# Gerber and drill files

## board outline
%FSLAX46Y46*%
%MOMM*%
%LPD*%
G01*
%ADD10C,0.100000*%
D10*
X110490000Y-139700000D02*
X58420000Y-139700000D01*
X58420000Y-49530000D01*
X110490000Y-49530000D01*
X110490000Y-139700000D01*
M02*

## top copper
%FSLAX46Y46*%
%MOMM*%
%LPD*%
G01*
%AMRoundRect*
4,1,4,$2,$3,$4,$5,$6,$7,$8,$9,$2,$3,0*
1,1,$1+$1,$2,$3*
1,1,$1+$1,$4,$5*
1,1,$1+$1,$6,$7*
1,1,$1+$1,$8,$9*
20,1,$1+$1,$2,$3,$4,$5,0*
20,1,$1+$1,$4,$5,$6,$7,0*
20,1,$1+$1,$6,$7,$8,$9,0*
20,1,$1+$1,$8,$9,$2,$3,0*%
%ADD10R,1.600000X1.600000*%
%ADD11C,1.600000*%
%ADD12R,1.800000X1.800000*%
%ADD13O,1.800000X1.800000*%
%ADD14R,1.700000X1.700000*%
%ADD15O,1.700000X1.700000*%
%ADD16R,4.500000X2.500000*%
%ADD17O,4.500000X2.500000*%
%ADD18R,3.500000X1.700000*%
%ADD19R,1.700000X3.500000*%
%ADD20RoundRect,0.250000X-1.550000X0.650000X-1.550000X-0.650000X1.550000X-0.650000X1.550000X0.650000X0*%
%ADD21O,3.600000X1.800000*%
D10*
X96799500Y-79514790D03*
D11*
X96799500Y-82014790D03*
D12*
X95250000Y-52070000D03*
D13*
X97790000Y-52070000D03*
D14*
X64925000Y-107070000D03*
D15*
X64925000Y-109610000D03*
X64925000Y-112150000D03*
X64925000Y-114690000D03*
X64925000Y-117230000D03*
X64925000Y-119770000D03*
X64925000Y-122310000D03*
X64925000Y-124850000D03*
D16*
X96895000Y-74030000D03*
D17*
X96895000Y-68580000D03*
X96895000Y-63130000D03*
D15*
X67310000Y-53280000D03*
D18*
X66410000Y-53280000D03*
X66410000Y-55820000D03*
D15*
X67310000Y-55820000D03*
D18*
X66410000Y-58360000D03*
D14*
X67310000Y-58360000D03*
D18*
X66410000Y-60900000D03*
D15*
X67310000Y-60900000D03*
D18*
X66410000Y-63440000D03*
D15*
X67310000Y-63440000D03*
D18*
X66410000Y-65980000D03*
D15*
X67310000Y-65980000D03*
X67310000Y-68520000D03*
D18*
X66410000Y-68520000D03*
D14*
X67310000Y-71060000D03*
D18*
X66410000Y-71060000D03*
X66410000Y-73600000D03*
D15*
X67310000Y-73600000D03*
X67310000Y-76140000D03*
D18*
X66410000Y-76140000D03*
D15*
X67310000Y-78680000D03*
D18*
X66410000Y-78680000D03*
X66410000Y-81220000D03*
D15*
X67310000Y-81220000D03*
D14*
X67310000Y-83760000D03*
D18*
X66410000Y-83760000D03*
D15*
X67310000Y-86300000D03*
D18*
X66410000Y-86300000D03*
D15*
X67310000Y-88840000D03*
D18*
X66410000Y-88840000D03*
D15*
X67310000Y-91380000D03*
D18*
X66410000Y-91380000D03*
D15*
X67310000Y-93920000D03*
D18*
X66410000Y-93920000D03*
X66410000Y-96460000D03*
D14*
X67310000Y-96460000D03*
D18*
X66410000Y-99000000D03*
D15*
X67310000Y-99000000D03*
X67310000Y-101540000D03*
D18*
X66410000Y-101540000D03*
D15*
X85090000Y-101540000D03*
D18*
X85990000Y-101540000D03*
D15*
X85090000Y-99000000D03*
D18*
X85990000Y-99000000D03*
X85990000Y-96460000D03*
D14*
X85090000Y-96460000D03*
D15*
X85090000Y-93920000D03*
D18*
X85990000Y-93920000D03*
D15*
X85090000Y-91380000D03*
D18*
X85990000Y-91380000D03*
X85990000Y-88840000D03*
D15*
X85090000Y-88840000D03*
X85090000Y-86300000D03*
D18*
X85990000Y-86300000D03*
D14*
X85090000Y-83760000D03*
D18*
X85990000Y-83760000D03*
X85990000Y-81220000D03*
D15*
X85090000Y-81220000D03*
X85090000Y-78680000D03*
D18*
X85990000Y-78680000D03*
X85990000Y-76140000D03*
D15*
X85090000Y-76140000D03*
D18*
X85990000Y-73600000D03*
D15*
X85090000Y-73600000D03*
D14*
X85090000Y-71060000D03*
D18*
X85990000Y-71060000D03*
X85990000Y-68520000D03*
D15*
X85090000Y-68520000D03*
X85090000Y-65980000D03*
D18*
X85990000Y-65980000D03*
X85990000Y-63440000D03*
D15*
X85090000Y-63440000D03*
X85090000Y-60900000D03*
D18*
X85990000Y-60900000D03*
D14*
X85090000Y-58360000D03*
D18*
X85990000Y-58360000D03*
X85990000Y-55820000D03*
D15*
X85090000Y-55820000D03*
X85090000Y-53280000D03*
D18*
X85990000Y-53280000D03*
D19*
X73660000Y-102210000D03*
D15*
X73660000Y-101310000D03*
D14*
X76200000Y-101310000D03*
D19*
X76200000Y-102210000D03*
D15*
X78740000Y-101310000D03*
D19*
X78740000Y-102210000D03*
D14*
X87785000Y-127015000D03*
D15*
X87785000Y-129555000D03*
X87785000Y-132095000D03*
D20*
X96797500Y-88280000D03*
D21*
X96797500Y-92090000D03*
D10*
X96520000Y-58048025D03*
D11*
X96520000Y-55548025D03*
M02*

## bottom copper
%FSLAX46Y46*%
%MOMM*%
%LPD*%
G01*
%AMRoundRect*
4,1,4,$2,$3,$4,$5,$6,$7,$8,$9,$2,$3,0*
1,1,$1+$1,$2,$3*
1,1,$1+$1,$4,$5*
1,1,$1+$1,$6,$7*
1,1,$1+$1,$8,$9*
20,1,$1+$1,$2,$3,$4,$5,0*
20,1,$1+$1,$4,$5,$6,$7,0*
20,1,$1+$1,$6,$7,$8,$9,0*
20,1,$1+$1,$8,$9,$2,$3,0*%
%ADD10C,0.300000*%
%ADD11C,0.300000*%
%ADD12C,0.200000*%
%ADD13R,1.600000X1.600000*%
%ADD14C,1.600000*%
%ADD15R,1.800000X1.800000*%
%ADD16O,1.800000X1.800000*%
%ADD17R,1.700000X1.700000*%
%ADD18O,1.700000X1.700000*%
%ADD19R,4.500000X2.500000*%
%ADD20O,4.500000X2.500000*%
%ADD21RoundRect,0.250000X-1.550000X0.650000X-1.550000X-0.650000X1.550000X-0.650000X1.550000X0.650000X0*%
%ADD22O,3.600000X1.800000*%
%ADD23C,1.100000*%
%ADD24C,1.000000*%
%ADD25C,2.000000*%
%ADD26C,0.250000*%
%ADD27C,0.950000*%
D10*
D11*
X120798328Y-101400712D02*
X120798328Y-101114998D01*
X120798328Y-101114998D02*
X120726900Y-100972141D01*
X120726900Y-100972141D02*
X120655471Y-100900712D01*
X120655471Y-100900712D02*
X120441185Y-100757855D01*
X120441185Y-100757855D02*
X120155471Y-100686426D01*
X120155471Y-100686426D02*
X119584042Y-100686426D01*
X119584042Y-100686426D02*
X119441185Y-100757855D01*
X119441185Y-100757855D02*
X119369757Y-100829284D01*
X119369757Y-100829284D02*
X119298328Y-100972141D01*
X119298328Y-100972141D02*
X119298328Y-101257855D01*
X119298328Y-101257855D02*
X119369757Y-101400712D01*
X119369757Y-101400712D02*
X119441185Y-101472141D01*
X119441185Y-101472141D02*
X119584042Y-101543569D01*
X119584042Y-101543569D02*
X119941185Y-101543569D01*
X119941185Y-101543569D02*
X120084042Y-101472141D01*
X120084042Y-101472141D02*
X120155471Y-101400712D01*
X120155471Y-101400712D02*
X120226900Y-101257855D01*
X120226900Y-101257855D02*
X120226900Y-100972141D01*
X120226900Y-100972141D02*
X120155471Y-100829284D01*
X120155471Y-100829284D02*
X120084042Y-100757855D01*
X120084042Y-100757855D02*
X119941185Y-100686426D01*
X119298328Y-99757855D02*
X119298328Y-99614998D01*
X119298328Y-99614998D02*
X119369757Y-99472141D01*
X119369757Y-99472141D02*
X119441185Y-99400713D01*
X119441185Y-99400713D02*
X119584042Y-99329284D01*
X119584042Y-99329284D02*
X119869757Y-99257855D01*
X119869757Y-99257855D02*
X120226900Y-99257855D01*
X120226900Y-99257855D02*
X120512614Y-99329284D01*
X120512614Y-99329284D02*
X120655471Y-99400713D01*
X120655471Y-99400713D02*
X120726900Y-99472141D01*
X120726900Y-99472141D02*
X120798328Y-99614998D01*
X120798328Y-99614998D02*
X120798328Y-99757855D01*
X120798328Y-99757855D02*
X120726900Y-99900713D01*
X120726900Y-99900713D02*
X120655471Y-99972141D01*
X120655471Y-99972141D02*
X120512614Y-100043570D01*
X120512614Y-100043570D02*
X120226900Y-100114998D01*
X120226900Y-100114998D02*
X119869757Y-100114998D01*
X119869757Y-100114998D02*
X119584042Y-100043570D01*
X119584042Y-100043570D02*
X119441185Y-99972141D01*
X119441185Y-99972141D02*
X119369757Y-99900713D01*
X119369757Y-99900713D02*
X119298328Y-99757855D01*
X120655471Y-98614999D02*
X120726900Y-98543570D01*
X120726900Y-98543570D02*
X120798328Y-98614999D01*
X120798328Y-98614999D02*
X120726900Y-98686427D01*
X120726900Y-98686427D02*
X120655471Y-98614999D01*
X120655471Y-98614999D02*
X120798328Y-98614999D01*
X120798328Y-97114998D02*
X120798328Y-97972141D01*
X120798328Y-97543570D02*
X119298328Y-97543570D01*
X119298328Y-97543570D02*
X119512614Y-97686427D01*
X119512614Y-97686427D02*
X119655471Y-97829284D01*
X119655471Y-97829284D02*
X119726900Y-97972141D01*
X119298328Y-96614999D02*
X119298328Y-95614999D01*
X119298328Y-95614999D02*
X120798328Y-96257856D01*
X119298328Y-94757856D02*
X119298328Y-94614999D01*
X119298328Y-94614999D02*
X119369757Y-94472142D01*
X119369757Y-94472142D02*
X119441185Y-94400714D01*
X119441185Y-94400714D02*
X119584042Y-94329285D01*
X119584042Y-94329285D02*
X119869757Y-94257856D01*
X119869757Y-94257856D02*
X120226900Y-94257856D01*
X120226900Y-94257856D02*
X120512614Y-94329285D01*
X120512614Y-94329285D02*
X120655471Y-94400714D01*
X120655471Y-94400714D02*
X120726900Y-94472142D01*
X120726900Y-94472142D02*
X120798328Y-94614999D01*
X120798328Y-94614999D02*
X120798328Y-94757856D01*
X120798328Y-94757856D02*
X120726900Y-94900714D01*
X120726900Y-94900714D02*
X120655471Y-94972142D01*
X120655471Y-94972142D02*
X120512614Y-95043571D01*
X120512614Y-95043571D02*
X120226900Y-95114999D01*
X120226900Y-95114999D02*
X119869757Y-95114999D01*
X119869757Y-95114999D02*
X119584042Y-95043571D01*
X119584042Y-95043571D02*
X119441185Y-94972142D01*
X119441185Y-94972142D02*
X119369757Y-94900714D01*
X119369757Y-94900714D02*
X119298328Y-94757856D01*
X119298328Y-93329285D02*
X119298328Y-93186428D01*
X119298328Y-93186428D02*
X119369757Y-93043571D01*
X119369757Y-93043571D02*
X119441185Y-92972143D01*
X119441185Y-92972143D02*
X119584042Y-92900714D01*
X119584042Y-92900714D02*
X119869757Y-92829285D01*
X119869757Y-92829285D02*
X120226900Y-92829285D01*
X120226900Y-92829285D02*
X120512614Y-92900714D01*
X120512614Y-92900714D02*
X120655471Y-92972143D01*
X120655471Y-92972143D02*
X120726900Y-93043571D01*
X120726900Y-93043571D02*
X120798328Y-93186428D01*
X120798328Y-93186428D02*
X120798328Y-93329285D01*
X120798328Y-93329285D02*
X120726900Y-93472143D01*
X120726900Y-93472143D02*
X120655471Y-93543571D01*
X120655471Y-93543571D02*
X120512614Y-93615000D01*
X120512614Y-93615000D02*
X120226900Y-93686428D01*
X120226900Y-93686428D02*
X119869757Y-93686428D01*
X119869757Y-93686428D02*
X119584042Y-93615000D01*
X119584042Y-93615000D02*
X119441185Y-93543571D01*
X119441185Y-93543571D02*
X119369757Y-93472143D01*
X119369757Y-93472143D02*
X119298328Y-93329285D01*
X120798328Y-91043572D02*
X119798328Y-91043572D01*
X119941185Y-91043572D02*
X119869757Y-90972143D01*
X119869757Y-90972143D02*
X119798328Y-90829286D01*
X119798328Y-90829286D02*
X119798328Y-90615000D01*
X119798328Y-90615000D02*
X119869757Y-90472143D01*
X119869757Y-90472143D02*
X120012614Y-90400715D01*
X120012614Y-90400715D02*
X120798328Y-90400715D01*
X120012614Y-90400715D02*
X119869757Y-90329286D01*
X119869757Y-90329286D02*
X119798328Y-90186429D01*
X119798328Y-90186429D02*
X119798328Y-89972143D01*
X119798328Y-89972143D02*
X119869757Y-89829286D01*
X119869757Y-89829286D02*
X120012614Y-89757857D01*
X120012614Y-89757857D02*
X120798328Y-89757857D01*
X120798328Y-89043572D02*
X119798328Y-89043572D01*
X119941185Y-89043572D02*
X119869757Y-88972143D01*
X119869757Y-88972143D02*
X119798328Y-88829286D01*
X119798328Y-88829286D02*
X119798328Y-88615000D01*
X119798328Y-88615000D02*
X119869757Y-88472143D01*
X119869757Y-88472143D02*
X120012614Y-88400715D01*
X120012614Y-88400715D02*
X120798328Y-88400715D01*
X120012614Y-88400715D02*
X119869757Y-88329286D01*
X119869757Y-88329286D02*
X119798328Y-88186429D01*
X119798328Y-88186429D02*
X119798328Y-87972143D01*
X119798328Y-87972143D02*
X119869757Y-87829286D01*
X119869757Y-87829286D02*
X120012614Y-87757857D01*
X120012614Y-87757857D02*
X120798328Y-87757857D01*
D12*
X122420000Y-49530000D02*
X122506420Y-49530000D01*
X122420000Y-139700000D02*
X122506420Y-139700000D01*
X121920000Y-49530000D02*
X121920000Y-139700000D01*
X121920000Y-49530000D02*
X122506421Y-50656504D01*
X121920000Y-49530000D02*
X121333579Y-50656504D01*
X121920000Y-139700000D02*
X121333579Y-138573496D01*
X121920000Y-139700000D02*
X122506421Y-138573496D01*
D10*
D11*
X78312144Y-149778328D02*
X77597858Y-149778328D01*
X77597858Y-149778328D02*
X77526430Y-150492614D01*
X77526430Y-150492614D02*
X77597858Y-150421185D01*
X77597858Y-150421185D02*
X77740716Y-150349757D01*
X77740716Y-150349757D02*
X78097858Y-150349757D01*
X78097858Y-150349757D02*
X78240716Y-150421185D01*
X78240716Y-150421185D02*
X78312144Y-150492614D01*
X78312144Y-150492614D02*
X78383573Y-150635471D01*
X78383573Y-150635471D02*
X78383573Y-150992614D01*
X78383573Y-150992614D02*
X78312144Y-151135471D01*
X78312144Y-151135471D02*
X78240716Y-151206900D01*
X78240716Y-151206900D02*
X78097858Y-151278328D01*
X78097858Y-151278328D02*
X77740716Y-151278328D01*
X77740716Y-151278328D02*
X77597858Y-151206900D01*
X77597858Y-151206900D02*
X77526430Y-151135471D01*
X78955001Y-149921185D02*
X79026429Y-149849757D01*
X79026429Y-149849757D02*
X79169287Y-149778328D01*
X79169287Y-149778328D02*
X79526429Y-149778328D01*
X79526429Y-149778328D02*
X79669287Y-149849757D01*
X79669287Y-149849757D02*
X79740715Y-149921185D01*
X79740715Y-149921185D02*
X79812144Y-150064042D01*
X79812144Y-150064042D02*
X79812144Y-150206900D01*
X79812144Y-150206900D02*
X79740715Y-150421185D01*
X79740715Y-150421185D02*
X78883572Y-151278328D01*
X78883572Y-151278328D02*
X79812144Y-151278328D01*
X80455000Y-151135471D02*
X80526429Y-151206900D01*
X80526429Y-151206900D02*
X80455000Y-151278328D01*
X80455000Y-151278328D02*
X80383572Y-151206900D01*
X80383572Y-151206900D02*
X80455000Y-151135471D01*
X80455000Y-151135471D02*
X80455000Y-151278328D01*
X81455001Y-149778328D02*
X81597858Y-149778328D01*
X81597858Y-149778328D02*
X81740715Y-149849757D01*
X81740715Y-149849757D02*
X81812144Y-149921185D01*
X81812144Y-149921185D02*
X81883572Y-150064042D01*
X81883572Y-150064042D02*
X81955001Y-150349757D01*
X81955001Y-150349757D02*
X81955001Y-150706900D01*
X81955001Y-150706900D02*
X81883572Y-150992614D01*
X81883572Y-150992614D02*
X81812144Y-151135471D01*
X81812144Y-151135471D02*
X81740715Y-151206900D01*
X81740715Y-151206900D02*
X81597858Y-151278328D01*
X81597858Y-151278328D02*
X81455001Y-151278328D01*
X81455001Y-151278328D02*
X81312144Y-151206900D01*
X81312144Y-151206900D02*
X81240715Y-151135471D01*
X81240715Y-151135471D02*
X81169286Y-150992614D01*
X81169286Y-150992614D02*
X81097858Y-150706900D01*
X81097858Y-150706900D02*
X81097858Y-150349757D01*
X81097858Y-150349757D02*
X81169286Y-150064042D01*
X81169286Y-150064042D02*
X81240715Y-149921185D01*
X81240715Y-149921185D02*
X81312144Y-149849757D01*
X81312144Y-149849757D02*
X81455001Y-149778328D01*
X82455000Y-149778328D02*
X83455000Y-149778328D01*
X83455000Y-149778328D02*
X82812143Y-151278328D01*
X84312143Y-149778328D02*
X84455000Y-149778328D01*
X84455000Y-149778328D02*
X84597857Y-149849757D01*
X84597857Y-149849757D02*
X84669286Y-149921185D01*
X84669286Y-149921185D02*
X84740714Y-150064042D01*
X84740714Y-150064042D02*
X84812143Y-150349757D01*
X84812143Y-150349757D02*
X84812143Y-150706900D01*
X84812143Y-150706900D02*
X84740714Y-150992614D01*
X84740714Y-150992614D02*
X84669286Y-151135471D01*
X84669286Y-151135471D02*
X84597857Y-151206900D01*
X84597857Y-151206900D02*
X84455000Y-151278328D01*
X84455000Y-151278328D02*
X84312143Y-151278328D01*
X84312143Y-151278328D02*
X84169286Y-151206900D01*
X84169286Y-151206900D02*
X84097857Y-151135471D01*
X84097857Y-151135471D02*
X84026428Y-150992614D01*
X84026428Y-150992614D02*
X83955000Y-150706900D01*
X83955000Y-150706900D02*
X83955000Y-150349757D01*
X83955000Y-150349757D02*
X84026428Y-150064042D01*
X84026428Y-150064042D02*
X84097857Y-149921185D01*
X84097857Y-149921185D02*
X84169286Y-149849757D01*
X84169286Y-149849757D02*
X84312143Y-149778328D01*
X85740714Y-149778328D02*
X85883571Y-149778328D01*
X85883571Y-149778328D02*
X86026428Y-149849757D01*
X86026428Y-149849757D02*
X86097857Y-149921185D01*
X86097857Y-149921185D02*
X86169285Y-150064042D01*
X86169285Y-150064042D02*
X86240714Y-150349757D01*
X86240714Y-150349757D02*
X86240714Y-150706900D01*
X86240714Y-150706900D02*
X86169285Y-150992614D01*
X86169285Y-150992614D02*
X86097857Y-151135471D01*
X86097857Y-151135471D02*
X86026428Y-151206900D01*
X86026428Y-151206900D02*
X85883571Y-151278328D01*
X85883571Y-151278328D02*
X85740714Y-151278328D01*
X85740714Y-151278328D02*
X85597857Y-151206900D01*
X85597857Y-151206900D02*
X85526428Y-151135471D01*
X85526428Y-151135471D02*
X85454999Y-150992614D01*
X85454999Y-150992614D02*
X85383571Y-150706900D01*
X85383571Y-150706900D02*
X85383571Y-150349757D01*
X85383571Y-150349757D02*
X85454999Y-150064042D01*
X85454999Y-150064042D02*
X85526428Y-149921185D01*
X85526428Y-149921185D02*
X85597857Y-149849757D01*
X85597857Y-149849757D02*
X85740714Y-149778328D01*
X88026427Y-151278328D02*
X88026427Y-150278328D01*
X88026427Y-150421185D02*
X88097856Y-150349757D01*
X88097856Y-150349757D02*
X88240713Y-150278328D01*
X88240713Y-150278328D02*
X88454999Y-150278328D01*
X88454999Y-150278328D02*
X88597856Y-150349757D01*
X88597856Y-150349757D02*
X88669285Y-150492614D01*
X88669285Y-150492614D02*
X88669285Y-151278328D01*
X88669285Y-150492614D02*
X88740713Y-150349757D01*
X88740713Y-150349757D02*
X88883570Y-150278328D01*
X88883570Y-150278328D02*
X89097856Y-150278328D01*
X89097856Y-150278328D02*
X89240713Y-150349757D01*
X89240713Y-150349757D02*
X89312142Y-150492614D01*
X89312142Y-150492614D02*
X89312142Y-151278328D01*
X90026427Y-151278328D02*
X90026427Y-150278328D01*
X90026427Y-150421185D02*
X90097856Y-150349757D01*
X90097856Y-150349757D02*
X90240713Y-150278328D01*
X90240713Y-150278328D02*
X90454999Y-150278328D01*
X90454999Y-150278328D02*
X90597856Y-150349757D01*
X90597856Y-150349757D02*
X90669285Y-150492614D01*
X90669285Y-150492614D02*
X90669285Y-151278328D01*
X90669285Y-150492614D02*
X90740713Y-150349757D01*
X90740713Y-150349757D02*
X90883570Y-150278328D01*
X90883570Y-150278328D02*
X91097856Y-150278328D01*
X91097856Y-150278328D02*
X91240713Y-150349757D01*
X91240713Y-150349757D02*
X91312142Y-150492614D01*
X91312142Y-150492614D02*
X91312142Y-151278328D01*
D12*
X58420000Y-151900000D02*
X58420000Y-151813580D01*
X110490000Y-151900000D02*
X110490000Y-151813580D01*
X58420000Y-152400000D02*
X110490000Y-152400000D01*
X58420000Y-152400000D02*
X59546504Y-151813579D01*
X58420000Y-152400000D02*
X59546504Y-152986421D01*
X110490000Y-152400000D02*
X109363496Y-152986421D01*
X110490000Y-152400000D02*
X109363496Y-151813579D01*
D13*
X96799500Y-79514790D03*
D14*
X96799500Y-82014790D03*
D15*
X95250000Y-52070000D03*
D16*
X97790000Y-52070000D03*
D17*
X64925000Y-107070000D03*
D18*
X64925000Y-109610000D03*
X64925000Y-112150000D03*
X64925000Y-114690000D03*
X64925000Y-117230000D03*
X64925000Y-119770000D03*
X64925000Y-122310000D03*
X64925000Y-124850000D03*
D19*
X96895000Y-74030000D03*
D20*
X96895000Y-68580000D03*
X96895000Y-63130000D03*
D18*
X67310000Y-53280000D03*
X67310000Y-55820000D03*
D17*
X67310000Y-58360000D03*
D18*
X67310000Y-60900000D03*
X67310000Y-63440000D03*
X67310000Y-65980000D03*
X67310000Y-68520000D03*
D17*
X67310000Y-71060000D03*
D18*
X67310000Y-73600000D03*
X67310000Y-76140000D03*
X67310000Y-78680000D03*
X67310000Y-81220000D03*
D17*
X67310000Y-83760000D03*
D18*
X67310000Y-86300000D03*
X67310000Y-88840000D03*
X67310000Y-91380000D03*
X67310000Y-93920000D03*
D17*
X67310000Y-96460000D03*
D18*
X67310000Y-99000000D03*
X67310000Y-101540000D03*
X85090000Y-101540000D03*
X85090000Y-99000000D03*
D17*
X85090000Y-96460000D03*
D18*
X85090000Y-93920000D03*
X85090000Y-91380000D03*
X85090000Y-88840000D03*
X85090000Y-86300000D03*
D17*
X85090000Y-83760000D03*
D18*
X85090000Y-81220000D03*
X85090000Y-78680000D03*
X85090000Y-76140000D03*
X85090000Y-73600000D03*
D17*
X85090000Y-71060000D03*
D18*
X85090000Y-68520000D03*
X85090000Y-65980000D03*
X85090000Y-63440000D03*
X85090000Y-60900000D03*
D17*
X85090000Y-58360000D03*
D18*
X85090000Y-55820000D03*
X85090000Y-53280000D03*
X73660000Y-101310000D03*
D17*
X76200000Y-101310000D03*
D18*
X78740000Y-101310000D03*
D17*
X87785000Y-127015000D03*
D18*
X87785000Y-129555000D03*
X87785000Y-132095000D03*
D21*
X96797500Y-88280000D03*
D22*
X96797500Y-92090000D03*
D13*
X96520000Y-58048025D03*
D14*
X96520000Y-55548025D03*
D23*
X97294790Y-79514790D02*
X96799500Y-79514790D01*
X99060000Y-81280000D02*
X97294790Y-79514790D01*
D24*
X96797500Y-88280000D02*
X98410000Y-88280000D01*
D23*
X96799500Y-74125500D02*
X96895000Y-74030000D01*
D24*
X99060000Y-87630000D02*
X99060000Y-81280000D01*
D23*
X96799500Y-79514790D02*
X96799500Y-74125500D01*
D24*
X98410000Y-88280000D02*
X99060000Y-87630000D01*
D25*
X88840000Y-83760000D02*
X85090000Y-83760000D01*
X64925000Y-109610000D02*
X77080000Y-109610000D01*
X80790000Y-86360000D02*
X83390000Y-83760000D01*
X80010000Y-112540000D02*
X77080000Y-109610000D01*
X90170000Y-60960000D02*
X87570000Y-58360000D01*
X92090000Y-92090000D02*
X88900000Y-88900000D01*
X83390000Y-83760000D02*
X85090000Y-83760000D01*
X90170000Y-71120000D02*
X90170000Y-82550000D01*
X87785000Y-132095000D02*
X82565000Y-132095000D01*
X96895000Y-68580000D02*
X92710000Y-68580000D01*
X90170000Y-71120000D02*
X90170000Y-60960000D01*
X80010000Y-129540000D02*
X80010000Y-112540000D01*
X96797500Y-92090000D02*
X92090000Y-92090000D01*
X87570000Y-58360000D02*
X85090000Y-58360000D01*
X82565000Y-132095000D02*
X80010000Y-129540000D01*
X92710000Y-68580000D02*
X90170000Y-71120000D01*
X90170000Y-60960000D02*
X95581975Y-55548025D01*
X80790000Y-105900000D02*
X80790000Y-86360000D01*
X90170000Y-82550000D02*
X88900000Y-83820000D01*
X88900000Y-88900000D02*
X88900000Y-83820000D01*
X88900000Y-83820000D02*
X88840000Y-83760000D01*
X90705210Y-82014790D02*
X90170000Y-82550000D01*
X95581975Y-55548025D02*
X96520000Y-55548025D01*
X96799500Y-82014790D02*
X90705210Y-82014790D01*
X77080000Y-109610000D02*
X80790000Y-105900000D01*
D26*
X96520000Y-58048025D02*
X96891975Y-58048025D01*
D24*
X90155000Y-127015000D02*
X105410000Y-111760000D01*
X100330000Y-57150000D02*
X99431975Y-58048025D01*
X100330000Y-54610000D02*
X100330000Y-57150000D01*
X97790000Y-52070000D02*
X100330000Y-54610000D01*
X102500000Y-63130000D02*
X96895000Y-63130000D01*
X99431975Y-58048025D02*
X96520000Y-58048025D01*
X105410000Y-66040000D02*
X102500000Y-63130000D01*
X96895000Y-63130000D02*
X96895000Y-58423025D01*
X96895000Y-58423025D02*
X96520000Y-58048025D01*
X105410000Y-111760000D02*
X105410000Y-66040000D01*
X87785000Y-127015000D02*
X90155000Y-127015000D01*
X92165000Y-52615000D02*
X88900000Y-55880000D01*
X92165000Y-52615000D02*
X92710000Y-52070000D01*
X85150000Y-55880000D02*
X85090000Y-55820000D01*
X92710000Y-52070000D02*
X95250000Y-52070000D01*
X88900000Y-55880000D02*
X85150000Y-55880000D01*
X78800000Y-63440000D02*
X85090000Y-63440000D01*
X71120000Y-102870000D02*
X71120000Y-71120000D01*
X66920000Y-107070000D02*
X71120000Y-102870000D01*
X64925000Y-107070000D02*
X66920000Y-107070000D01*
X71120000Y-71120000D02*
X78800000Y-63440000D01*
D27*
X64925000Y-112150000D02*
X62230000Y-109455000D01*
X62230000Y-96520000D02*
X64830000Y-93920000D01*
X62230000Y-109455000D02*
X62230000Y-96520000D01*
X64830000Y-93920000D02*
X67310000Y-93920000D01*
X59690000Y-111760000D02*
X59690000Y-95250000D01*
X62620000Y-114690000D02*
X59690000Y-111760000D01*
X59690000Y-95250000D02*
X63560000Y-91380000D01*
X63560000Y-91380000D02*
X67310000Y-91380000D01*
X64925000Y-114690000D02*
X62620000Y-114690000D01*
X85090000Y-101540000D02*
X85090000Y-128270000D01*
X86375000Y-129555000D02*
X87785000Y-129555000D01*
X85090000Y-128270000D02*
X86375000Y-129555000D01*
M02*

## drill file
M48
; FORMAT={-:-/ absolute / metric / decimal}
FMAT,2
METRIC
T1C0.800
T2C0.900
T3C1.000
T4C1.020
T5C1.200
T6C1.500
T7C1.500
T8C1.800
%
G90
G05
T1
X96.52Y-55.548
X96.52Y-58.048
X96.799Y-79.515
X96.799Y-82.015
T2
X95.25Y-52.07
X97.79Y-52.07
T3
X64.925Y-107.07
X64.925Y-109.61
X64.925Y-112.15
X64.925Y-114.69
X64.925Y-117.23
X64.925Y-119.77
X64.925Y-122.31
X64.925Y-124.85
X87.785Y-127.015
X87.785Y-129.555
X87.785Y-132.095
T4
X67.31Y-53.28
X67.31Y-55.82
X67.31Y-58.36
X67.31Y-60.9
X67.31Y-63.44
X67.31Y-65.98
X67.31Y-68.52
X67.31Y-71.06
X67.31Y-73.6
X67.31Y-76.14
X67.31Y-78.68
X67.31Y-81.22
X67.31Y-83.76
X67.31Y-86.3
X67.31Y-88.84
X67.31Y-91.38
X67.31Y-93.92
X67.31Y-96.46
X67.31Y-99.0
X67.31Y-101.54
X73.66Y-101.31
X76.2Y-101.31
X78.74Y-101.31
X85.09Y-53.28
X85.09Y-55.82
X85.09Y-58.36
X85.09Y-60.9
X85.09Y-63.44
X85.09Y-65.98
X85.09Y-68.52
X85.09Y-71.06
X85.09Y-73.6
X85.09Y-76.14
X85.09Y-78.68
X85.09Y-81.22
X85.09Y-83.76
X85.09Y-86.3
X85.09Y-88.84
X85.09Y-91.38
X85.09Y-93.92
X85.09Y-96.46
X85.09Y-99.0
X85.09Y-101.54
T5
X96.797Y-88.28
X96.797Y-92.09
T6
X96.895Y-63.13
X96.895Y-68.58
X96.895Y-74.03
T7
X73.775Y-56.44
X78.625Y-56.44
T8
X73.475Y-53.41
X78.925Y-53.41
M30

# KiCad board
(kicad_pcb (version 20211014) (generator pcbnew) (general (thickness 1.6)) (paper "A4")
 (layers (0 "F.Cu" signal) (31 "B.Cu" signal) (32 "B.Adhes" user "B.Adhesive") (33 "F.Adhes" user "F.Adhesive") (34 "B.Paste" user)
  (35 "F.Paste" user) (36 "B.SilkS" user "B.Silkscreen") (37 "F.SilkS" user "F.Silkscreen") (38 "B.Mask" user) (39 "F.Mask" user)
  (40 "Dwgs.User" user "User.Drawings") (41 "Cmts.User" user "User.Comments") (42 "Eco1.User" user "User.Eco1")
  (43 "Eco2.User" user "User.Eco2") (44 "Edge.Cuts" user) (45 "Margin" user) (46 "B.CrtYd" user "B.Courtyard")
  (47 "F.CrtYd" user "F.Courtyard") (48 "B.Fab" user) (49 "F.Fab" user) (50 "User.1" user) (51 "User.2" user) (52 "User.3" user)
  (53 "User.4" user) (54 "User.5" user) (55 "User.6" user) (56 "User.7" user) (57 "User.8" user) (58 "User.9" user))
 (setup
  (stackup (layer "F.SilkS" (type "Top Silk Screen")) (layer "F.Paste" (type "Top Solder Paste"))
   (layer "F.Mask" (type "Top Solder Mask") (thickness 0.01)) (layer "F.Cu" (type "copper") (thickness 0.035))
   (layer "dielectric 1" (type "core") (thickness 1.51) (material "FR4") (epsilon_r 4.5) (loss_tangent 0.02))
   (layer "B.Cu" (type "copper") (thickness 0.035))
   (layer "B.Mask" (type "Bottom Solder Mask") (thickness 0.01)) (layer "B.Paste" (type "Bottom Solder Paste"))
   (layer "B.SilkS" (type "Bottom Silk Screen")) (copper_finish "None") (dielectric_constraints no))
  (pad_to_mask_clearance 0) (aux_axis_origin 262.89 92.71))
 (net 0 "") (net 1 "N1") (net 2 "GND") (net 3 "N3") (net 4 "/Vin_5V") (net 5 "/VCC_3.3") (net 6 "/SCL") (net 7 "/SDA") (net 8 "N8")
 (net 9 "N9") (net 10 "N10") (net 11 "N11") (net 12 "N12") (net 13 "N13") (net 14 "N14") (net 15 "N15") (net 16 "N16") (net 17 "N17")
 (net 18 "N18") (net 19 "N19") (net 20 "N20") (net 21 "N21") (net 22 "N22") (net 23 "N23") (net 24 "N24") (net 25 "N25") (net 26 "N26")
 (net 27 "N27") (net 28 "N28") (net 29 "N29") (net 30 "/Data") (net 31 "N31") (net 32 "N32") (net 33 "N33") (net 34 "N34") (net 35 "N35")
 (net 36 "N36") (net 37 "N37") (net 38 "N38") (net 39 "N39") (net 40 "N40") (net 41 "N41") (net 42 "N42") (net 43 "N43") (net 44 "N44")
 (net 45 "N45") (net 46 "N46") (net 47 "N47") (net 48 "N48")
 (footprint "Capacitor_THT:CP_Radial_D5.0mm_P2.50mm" (layer "F.Cu") (at 96.7995 79.51479 -90)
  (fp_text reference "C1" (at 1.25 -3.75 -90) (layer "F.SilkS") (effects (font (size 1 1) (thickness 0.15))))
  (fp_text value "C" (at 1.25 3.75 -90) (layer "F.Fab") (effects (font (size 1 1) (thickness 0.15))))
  (pad "1" thru_hole rect (at 0 0 270) (size 1.6 1.6) (drill 0.8) (layers *.Cu *.Mask) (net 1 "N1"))
  (pad "2" thru_hole circle (at 2.5 0 270) (size 1.6 1.6) (drill 0.8) (layers *.Cu *.Mask) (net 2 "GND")))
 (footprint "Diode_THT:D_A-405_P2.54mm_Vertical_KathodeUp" (layer "F.Cu") (at 95.25 52.07)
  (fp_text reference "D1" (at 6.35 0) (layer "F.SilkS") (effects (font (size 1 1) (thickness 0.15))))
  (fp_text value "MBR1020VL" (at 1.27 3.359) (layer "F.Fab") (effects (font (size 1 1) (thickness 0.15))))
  (pad "1" thru_hole rect (at 0 0) (size 1.8 1.8) (drill 0.9) (layers *.Cu *.Mask) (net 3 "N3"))
  (pad "2" thru_hole oval (at 2.54 0) (size 1.8 1.8) (drill 0.9) (layers *.Cu *.Mask) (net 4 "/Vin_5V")))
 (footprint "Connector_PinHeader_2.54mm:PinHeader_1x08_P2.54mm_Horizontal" (layer "F.Cu") (at 64.925 107.07)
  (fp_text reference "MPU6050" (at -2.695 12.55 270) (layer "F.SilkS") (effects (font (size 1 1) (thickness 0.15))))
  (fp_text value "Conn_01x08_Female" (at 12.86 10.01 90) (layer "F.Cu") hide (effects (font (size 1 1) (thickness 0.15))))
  (pad "1" thru_hole rect (at 0 0) (size 1.7 1.7) (drill 1) (layers *.Cu *.Mask) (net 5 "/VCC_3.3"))
  (pad "2" thru_hole oval (at 0 2.54) (size 1.7 1.7) (drill 1) (layers *.Cu *.Mask) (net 2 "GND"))
  (pad "3" thru_hole oval (at 0 5.08) (size 1.7 1.7) (drill 1) (layers *.Cu *.Mask) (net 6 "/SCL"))
  (pad "4" thru_hole oval (at 0 7.62) (size 1.7 1.7) (drill 1) (layers *.Cu *.Mask) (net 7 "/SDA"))
  (pad "5" thru_hole oval (at 0 10.16) (size 1.7 1.7) (drill 1) (layers *.Cu *.Mask) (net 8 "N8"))
  (pad "6" thru_hole oval (at 0 12.7) (size 1.7 1.7) (drill 1) (layers *.Cu *.Mask) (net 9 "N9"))
  (pad "7" thru_hole oval (at 0 15.24) (size 1.7 1.7) (drill 1) (layers *.Cu *.Mask) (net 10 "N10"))
  (pad "8" thru_hole oval (at 0 17.78) (size 1.7 1.7) (drill 1) (layers *.Cu *.Mask) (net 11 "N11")))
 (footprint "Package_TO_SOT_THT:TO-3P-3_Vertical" (layer "F.Cu") (at 96.895 74.03 90)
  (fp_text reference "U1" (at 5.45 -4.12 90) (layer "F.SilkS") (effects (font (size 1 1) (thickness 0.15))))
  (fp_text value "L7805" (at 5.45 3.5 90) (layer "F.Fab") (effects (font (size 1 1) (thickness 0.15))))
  (pad "1" thru_hole rect (at 0 0 90) (size 2.5 4.5) (drill 1.5) (layers *.Cu *.Mask) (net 1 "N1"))
  (pad "2" thru_hole oval (at 5.45 0 90) (size 2.5 4.5) (drill 1.5) (layers *.Cu *.Mask) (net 2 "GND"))
  (pad "3" thru_hole oval (at 10.9 0 90) (size 2.5 4.5) (drill 1.5) (layers *.Cu *.Mask) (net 4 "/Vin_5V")))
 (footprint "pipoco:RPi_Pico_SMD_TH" (layer "F.Cu") (at 76.2 77.41)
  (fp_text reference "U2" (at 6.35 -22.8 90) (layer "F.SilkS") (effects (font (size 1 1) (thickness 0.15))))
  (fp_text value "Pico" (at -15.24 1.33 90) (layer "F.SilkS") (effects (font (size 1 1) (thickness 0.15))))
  (pad "" np_thru_hole oval (at -2.425 -20.97) (size 1.5 1.5) (drill 1.5) (layers *.Cu *.Mask))
  (pad "" np_thru_hole oval (at -2.725 -24) (size 1.8 1.8) (drill 1.8) (layers *.Cu *.Mask))
  (pad "" np_thru_hole oval (at 2.725 -24) (size 1.8 1.8) (drill 1.8) (layers *.Cu *.Mask))
  (pad "" np_thru_hole oval (at 2.425 -20.97) (size 1.5 1.5) (drill 1.5) (layers *.Cu *.Mask))
  (pad "1" thru_hole oval (at -8.89 -24.13) (size 1.7 1.7) (drill 1.02) (layers *.Cu *.Mask) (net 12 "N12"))
  (pad "1" smd rect (at -8.89 -24.13) (size 3.5 1.7) (drill (offset -0.9 0)) (layers "F.Cu" "F.Mask") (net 12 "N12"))
  (pad "2" smd rect (at -8.89 -21.59) (size 3.5 1.7) (drill (offset -0.9 0)) (layers "F.Cu" "F.Mask") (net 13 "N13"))
  (pad "2" thru_hole oval (at -8.89 -21.59) (size 1.7 1.7) (drill 1.02) (layers *.Cu *.Mask) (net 13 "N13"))
  (pad "3" smd rect (at -8.89 -19.05) (size 3.5 1.7) (drill (offset -0.9 0)) (layers "F.Cu" "F.Mask") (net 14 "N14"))
  (pad "3" thru_hole rect (at -8.89 -19.05) (size 1.7 1.7) (drill 1.02) (layers *.Cu *.Mask) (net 14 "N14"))
  (pad "4" smd rect (at -8.89 -16.51) (size 3.5 1.7) (drill (offset -0.9 0)) (layers "F.Cu" "F.Mask") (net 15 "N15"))
  (pad "4" thru_hole oval (at -8.89 -16.51) (size 1.7 1.7) (drill 1.02) (layers *.Cu *.Mask) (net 15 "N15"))
  (pad "5" smd rect (at -8.89 -13.97) (size 3.5 1.7) (drill (offset -0.9 0)) (layers "F.Cu" "F.Mask") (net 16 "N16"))
  (pad "5" thru_hole oval (at -8.89 -13.97) (size 1.7 1.7) (drill 1.02) (layers *.Cu *.Mask) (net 16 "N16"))
  (pad "6" smd rect (at -8.89 -11.43) (size 3.5 1.7) (drill (offset -0.9 0)) (layers "F.Cu" "F.Mask") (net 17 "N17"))
  (pad "6" thru_hole oval (at -8.89 -11.43) (size 1.7 1.7) (drill 1.02) (layers *.Cu *.Mask) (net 17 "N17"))
  (pad "7" thru_hole oval (at -8.89 -8.89) (size 1.7 1.7) (drill 1.02) (layers *.Cu *.Mask) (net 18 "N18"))
  (pad "7" smd rect (at -8.89 -8.89) (size 3.5 1.7) (drill (offset -0.9 0)) (layers "F.Cu" "F.Mask") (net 18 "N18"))
  (pad "8" thru_hole rect (at -8.89 -6.35) (size 1.7 1.7) (drill 1.02) (layers *.Cu *.Mask) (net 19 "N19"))
  (pad "8" smd rect (at -8.89 -6.35) (size 3.5 1.7) (drill (offset -0.9 0)) (layers "F.Cu" "F.Mask") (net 19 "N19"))
  (pad "9" smd rect (at -8.89 -3.81) (size 3.5 1.7) (drill (offset -0.9 0)) (layers "F.Cu" "F.Mask") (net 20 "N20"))
  (pad "9" thru_hole oval (at -8.89 -3.81) (size 1.7 1.7) (drill 1.02) (layers *.Cu *.Mask) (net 20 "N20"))
  (pad "10" thru_hole oval (at -8.89 -1.27) (size 1.7 1.7) (drill 1.02) (layers *.Cu *.Mask) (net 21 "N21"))
  (pad "10" smd rect (at -8.89 -1.27) (size 3.5 1.7) (drill (offset -0.9 0)) (layers "F.Cu" "F.Mask") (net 21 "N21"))
  (pad "11" thru_hole oval (at -8.89 1.27) (size 1.7 1.7) (drill 1.02) (layers *.Cu *.Mask) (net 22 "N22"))
  (pad "11" smd rect (at -8.89 1.27) (size 3.5 1.7) (drill (offset -0.9 0)) (layers "F.Cu" "F.Mask") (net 22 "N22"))
  (pad "12" smd rect (at -8.89 3.81) (size 3.5 1.7) (drill (offset -0.9 0)) (layers "F.Cu" "F.Mask") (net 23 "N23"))
  (pad "12" thru_hole oval (at -8.89 3.81) (size 1.7 1.7) (drill 1.02) (layers *.Cu *.Mask) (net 23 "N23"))
  (pad "13" thru_hole rect (at -8.89 6.35) (size 1.7 1.7) (drill 1.02) (layers *.Cu *.Mask) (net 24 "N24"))
  (pad "13" smd rect (at -8.89 6.35) (size 3.5 1.7) (drill (offset -0.9 0)) (layers "F.Cu" "F.Mask") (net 24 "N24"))
  (pad "14" thru_hole oval (at -8.89 8.89) (size 1.7 1.7) (drill 1.02) (layers *.Cu *.Mask) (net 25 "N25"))
  (pad "14" smd rect (at -8.89 8.89) (size 3.5 1.7) (drill (offset -0.9 0)) (layers "F.Cu" "F.Mask") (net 25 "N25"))
  (pad "15" thru_hole oval (at -8.89 11.43) (size 1.7 1.7) (drill 1.02) (layers *.Cu *.Mask) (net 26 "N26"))
  (pad "15" smd rect (at -8.89 11.43) (size 3.5 1.7) (drill (offset -0.9 0)) (layers "F.Cu" "F.Mask") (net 26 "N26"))
  (pad "16" thru_hole oval (at -8.89 13.97) (size 1.7 1.7) (drill 1.02) (layers *.Cu *.Mask) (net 7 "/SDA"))
  (pad "16" smd rect (at -8.89 13.97) (size 3.5 1.7) (drill (offset -0.9 0)) (layers "F.Cu" "F.Mask") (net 7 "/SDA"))
  (pad "17" thru_hole oval (at -8.89 16.51) (size 1.7 1.7) (drill 1.02) (layers *.Cu *.Mask) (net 6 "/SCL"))
  (pad "17" smd rect (at -8.89 16.51) (size 3.5 1.7) (drill (offset -0.9 0)) (layers "F.Cu" "F.Mask") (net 6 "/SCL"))
  (pad "18" smd rect (at -8.89 19.05) (size 3.5 1.7) (drill (offset -0.9 0)) (layers "F.Cu" "F.Mask") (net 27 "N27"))
  (pad "18" thru_hole rect (at -8.89 19.05) (size 1.7 1.7) (drill 1.02) (layers *.Cu *.Mask) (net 27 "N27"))
  (pad "19" smd rect (at -8.89 21.59) (size 3.5 1.7) (drill (offset -0.9 0)) (layers "F.Cu" "F.Mask") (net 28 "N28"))
  (pad "19" thru_hole oval (at -8.89 21.59) (size 1.7 1.7) (drill 1.02) (layers *.Cu *.Mask) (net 28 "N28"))
  (pad "20" thru_hole oval (at -8.89 24.13) (size 1.7 1.7) (drill 1.02) (layers *.Cu *.Mask) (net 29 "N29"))
  (pad "20" smd rect (at -8.89 24.13) (size 3.5 1.7) (drill (offset -0.9 0)) (layers "F.Cu" "F.Mask") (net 29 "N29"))
  (pad "21" thru_hole oval (at 8.89 24.13) (size 1.7 1.7) (drill 1.02) (layers *.Cu *.Mask) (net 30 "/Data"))
  (pad "21" smd rect (at 8.89 24.13) (size 3.5 1.7) (drill (offset 0.9 0)) (layers "F.Cu" "F.Mask") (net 30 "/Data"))
  (pad "22" thru_hole oval (at 8.89 21.59) (size 1.7 1.7) (drill 1.02) (layers *.Cu *.Mask) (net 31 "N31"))
  (pad "22" smd rect (at 8.89 21.59) (size 3.5 1.7) (drill (offset 0.9 0)) (layers "F.Cu" "F.Mask") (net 31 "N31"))
  (pad "23" smd rect (at 8.89 19.05) (size 3.5 1.7) (drill (offset 0.9 0)) (layers "F.Cu" "F.Mask") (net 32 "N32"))
  (pad "23" thru_hole rect (at 8.89 19.05) (size 1.7 1.7) (drill 1.02) (layers *.Cu *.Mask) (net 32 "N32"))
  (pad "24" thru_hole oval (at 8.89 16.51) (size 1.7 1.7) (drill 1.02) (layers *.Cu *.Mask) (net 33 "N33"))
  (pad "24" smd rect (at 8.89 16.51) (size 3.5 1.7) (drill (offset 0.9 0)) (layers "F.Cu" "F.Mask") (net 33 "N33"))
  (pad "25" thru_hole oval (at 8.89 13.97) (size 1.7 1.7) (drill 1.02) (layers *.Cu *.Mask) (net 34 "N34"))
  (pad "25" smd rect (at 8.89 13.97) (size 3.5 1.7) (drill (offset 0.9 0)) (layers "F.Cu" "F.Mask") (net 34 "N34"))
  (pad "26" smd rect (at 8.89 11.43) (size 3.5 1.7) (drill (offset 0.9 0)) (layers "F.Cu" "F.Mask") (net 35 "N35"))
  (pad "26" thru_hole oval (at 8.89 11.43) (size 1.7 1.7) (drill 1.02) (layers *.Cu *.Mask) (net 35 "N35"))
  (pad "27" thru_hole oval (at 8.89 8.89) (size 1.7 1.7) (drill 1.02) (layers *.Cu *.Mask) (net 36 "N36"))
  (pad "27" smd rect (at 8.89 8.89) (size 3.5 1.7) (drill (offset 0.9 0)) (layers "F.Cu" "F.Mask") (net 36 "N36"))
  (pad "28" thru_hole rect (at 8.89 6.35) (size 1.7 1.7) (drill 1.02) (layers *.Cu *.Mask) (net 2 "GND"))
  (pad "28" smd rect (at 8.89 6.35) (size 3.5 1.7) (drill (offset 0.9 0)) (layers "F.Cu" "F.Mask") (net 2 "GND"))
  (pad "29" smd rect (at 8.89 3.81) (size 3.5 1.7) (drill (offset 0.9 0)) (layers "F.Cu" "F.Mask") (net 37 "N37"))
  (pad "29" thru_hole oval (at 8.89 3.81) (size 1.7 1.7) (drill 1.02) (layers *.Cu *.Mask) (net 37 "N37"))
  (pad "30" thru_hole oval (at 8.89 1.27) (size 1.7 1.7) (drill 1.02) (layers *.Cu *.Mask) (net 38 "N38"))
  (pad "30" smd rect (at 8.89 1.27) (size 3.5 1.7) (drill (offset 0.9 0)) (layers "F.Cu" "F.Mask") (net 38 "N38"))
  (pad "31" smd rect (at 8.89 -1.27) (size 3.5 1.7) (drill (offset 0.9 0)) (layers "F.Cu" "F.Mask") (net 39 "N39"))
  (pad "31" thru_hole oval (at 8.89 -1.27) (size 1.7 1.7) (drill 1.02) (layers *.Cu *.Mask) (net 39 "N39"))
  (pad "32" smd rect (at 8.89 -3.81) (size 3.5 1.7) (drill (offset 0.9 0)) (layers "F.Cu" "F.Mask") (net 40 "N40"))
  (pad "32" thru_hole oval (at 8.89 -3.81) (size 1.7 1.7) (drill 1.02) (layers *.Cu *.Mask) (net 40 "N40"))
  (pad "33" thru_hole rect (at 8.89 -6.35) (size 1.7 1.7) (drill 1.02) (layers *.Cu *.Mask) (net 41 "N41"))
  (pad "33" smd rect (at 8.89 -6.35) (size 3.5 1.7) (drill (offset 0.9 0)) (layers "F.Cu" "F.Mask") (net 41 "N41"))
  (pad "34" smd rect (at 8.89 -8.89) (size 3.5 1.7) (drill (offset 0.9 0)) (layers "F.Cu" "F.Mask") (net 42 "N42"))
  (pad "34" thru_hole oval (at 8.89 -8.89) (size 1.7 1.7) (drill 1.02) (layers *.Cu *.Mask) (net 42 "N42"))
  (pad "35" thru_hole oval (at 8.89 -11.43) (size 1.7 1.7) (drill 1.02) (layers *.Cu *.Mask) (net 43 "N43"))
  (pad "35" smd rect (at 8.89 -11.43) (size 3.5 1.7) (drill (offset 0.9 0)) (layers "F.Cu" "F.Mask") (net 43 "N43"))
  (pad "36" smd rect (at 8.89 -13.97) (size 3.5 1.7) (drill (offset 0.9 0)) (layers "F.Cu" "F.Mask") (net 5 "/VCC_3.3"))
  (pad "36" thru_hole oval (at 8.89 -13.97) (size 1.7 1.7) (drill 1.02) (layers *.Cu *.Mask) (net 5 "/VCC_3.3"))
  (pad "37" thru_hole oval (at 8.89 -16.51) (size 1.7 1.7) (drill 1.02) (layers *.Cu *.Mask) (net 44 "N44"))
  (pad "37" smd rect (at 8.89 -16.51) (size 3.5 1.7) (drill (offset 0.9 0)) (layers "F.Cu" "F.Mask") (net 44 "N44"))
  (pad "38" thru_hole rect (at 8.89 -19.05) (size 1.7 1.7) (drill 1.02) (layers *.Cu *.Mask) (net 2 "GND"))
  (pad "38" smd rect (at 8.89 -19.05) (size 3.5 1.7) (drill (offset 0.9 0)) (layers "F.Cu" "F.Mask") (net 2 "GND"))
  (pad "39" smd rect (at 8.89 -21.59) (size 3.5 1.7) (drill (offset 0.9 0)) (layers "F.Cu" "F.Mask") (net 3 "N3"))
  (pad "39" thru_hole oval (at 8.89 -21.59) (size 1.7 1.7) (drill 1.02) (layers *.Cu *.Mask) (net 3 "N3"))
  (pad "40" thru_hole oval (at 8.89 -24.13) (size 1.7 1.7) (drill 1.02) (layers *.Cu *.Mask) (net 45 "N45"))
  (pad "40" smd rect (at 8.89 -24.13) (size 3.5 1.7) (drill (offset 0.9 0)) (layers "F.Cu" "F.Mask") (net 45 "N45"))
  (pad "41" smd rect (at -2.54 23.9 90) (size 3.5 1.7) (drill (offset -0.9 0)) (layers "F.Cu" "F.Mask") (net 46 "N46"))
  (pad "41" thru_hole oval (at -2.54 23.9) (size 1.7 1.7) (drill 1.02) (layers *.Cu *.Mask) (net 46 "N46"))
  (pad "42" thru_hole rect (at 0 23.9) (size 1.7 1.7) (drill 1.02) (layers *.Cu *.Mask) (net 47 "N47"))
  (pad "42" smd rect (at 0 23.9 90) (size 3.5 1.7) (drill (offset -0.9 0)) (layers "F.Cu" "F.Mask") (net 47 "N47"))
  (pad "43" thru_hole oval (at 2.54 23.9) (size 1.7 1.7) (drill 1.02) (layers *.Cu *.Mask) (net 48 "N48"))
  (pad "43" smd rect (at 2.54 23.9 90) (size 3.5 1.7) (drill (offset -0.9 0)) (layers "F.Cu" "F.Mask") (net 48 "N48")))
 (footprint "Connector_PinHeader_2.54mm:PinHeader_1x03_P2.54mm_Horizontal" (layer "F.Cu") (at 87.785 127.015)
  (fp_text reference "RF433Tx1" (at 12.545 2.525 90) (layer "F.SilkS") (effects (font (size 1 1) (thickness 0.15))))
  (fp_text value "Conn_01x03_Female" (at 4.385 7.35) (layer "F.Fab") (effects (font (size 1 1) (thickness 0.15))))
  (pad "1" thru_hole rect (at 0 0) (size 1.7 1.7) (drill 1) (layers *.Cu *.Mask) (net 4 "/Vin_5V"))
  (pad "2" thru_hole oval (at 0 2.54) (size 1.7 1.7) (drill 1) (layers *.Cu *.Mask) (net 30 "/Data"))
  (pad "3" thru_hole oval (at 0 5.08) (size 1.7 1.7) (drill 1) (layers *.Cu *.Mask) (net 2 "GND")))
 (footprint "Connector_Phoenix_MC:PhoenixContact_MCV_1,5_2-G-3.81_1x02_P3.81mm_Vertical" (layer "F.Cu") (at 96.7975 88.28 -90)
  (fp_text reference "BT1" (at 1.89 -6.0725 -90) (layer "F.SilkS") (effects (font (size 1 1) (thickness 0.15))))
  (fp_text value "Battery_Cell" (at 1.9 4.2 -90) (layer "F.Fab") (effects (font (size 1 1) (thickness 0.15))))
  (pad "1" thru_hole roundrect (at 0 0 270) (size 1.8 3.6) (drill 1.2) (layers *.Cu *.Mask) (roundrect_rratio 0.138889) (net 1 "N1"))
  (pad "2" thru_hole oval (at 3.81 0 270) (size 1.8 3.6) (drill 1.2) (layers *.Cu *.Mask) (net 2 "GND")))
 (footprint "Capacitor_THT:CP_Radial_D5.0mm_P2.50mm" (layer "F.Cu") (at 96.52 58.048025 90)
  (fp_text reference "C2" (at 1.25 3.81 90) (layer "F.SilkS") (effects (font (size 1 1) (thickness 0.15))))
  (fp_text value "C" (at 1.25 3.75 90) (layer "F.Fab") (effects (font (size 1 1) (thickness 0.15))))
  (pad "1" thru_hole rect (at 0 0 90) (size 1.6 1.6) (drill 0.8) (layers *.Cu *.Mask) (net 4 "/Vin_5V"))
  (pad "2" thru_hole circle (at 2.5 0 90) (size 1.6 1.6) (drill 0.8) (layers *.Cu *.Mask) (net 2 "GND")))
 (gr_poly (pts (xy 110.49 139.7) (xy 58.42 139.7) (xy 58.42 49.53) (xy 110.49 49.53)) (layer "Edge.Cuts") (width 0.1) (fill none))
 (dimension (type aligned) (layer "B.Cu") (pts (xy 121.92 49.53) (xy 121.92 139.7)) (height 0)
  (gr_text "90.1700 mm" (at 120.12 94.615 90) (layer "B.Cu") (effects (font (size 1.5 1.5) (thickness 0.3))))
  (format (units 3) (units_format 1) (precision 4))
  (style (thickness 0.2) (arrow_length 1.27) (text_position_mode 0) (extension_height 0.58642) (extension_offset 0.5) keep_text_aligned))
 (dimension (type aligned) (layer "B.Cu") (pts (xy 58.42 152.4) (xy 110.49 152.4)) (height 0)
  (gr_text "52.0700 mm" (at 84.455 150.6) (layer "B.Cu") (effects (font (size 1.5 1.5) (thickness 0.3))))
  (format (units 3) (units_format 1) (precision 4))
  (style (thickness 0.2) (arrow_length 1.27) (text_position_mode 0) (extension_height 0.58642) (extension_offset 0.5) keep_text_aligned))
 (segment (start 97.29479 79.51479) (end 96.7995 79.51479) (width 1.1) (layer "B.Cu") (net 1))
 (segment (start 99.06 81.28) (end 97.29479 79.51479) (width 1.1) (layer "B.Cu") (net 1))
 (segment (start 96.7975 88.28) (end 98.41 88.28) (width 1) (layer "B.Cu") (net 1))
 (segment (start 96.7995 74.1255) (end 96.895 74.03) (width 1.1) (layer "B.Cu") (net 1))
 (segment (start 99.06 87.63) (end 99.06 81.28) (width 1) (layer "B.Cu") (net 1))
 (segment (start 96.7995 79.51479) (end 96.7995 74.1255) (width 1.1) (layer "B.Cu") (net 1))
 (segment (start 98.41 88.28) (end 99.06 87.63) (width 1) (layer "B.Cu") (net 1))
 (segment (start 88.84 83.76) (end 85.09 83.76) (width 2) (layer "B.Cu") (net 2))
 (segment (start 64.925 109.61) (end 77.08 109.61) (width 2) (layer "B.Cu") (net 2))
 (segment (start 80.79 86.36) (end 83.39 83.76) (width 2) (layer "B.Cu") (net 2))
 (segment (start 80.01 112.54) (end 77.08 109.61) (width 2) (layer "B.Cu") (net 2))
 (segment (start 90.17 60.96) (end 87.57 58.36) (width 2) (layer "B.Cu") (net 2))
 (segment (start 92.09 92.09) (end 88.9 88.9) (width 2) (layer "B.Cu") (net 2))
 (segment (start 83.39 83.76) (end 85.09 83.76) (width 2) (layer "B.Cu") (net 2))
 (segment (start 90.17 71.12) (end 90.17 82.55) (width 2) (layer "B.Cu") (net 2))
 (segment (start 87.785 132.095) (end 82.565 132.095) (width 2) (layer "B.Cu") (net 2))
 (segment (start 96.895 68.58) (end 92.71 68.58) (width 2) (layer "B.Cu") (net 2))
 (segment (start 90.17 71.12) (end 90.17 60.96) (width 2) (layer "B.Cu") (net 2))
 (segment (start 80.01 129.54) (end 80.01 112.54) (width 2) (layer "B.Cu") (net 2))
 (segment (start 96.7975 92.09) (end 92.09 92.09) (width 2) (layer "B.Cu") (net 2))
 (segment (start 87.57 58.36) (end 85.09 58.36) (width 2) (layer "B.Cu") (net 2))
 (segment (start 82.565 132.095) (end 80.01 129.54) (width 2) (layer "B.Cu") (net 2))
 (segment (start 92.71 68.58) (end 90.17 71.12) (width 2) (layer "B.Cu") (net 2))
 (segment (start 90.17 60.96) (end 95.581975 55.548025) (width 2) (layer "B.Cu") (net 2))
 (segment (start 80.79 105.9) (end 80.79 86.36) (width 2) (layer "B.Cu") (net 2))
 (segment (start 90.17 82.55) (end 88.9 83.82) (width 2) (layer "B.Cu") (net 2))
 (segment (start 88.9 88.9) (end 88.9 83.82) (width 2) (layer "B.Cu") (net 2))
 (segment (start 88.9 83.82) (end 88.84 83.76) (width 2) (layer "B.Cu") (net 2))
 (segment (start 90.70521 82.01479) (end 90.17 82.55) (width 2) (layer "B.Cu") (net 2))
 (segment (start 95.581975 55.548025) (end 96.52 55.548025) (width 2) (layer "B.Cu") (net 2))
 (segment (start 96.7995 82.01479) (end 90.70521 82.01479) (width 2) (layer "B.Cu") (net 2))
 (segment (start 77.08 109.61) (end 80.79 105.9) (width 2) (layer "B.Cu") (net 2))
 (segment (start 96.52 58.048025) (end 96.891975 58.048025) (width 0.25) (layer "B.Cu") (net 4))
 (segment (start 90.155 127.015) (end 105.41 111.76) (width 1) (layer "B.Cu") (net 4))
 (segment (start 100.33 57.15) (end 99.431975 58.048025) (width 1) (layer "B.Cu") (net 4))
 (segment (start 100.33 54.61) (end 100.33 57.15) (width 1) (layer "B.Cu") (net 4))
 (segment (start 97.79 52.07) (end 100.33 54.61) (width 1) (layer "B.Cu") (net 4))
 (segment (start 102.5 63.13) (end 96.895 63.13) (width 1) (layer "B.Cu") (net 4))
 (segment (start 99.431975 58.048025) (end 96.52 58.048025) (width 1) (layer "B.Cu") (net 4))
 (segment (start 105.41 66.04) (end 102.5 63.13) (width 1) (layer "B.Cu") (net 4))
 (segment (start 96.895 63.13) (end 96.895 58.423025) (width 1) (layer "B.Cu") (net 4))
 (segment (start 96.895 58.423025) (end 96.52 58.048025) (width 1) (layer "B.Cu") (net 4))
 (segment (start 105.41 111.76) (end 105.41 66.04) (width 1) (layer "B.Cu") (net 4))
 (segment (start 87.785 127.015) (end 90.155 127.015) (width 1) (layer "B.Cu") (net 4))
 (segment (start 92.165 52.615) (end 88.9 55.88) (width 1) (layer "B.Cu") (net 3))
 (segment (start 92.165 52.615) (end 92.71 52.07) (width 1) (layer "B.Cu") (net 3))
 (segment (start 85.15 55.88) (end 85.09 55.82) (width 1) (layer "B.Cu") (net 3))
 (segment (start 92.71 52.07) (end 95.25 52.07) (width 1) (layer "B.Cu") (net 3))
 (segment (start 88.9 55.88) (end 85.15 55.88) (width 1) (layer "B.Cu") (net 3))
 (segment (start 78.8 63.44) (end 85.09 63.44) (width 1) (layer "B.Cu") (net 5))
 (segment (start 71.12 102.87) (end 71.12 71.12) (width 1) (layer "B.Cu") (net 5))
 (segment (start 66.92 107.07) (end 71.12 102.87) (width 1) (layer "B.Cu") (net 5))
 (segment (start 64.925 107.07) (end 66.92 107.07) (width 1) (layer "B.Cu") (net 5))
 (segment (start 71.12 71.12) (end 78.8 63.44) (width 1) (layer "B.Cu") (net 5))
 (segment (start 64.925 112.15) (end 62.23 109.455) (width 0.95) (layer "B.Cu") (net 6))
 (segment (start 62.23 96.52) (end 64.83 93.92) (width 0.95) (layer "B.Cu") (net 6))
 (segment (start 62.23 109.455) (end 62.23 96.52) (width 0.95) (layer "B.Cu") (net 6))
 (segment (start 64.83 93.92) (end 67.31 93.92) (width 0.95) (layer "B.Cu") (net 6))
 (segment (start 59.69 111.76) (end 59.69 95.25) (width 0.95) (layer "B.Cu") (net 7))
 (segment (start 62.62 114.69) (end 59.69 111.76) (width 0.95) (layer "B.Cu") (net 7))
 (segment (start 59.69 95.25) (end 63.56 91.38) (width 0.95) (layer "B.Cu") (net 7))
 (segment (start 63.56 91.38) (end 67.31 91.38) (width 0.95) (layer "B.Cu") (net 7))
 (segment (start 64.925 114.69) (end 62.62 114.69) (width 0.95) (layer "B.Cu") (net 7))
 (segment (start 85.09 101.54) (end 85.09 128.27) (width 0.95) (layer "B.Cu") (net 30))
 (segment (start 86.375 129.555) (end 87.785 129.555) (width 0.95) (layer "B.Cu") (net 30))
 (segment (start 85.09 128.27) (end 86.375 129.555) (width 0.95) (layer "B.Cu") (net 30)))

